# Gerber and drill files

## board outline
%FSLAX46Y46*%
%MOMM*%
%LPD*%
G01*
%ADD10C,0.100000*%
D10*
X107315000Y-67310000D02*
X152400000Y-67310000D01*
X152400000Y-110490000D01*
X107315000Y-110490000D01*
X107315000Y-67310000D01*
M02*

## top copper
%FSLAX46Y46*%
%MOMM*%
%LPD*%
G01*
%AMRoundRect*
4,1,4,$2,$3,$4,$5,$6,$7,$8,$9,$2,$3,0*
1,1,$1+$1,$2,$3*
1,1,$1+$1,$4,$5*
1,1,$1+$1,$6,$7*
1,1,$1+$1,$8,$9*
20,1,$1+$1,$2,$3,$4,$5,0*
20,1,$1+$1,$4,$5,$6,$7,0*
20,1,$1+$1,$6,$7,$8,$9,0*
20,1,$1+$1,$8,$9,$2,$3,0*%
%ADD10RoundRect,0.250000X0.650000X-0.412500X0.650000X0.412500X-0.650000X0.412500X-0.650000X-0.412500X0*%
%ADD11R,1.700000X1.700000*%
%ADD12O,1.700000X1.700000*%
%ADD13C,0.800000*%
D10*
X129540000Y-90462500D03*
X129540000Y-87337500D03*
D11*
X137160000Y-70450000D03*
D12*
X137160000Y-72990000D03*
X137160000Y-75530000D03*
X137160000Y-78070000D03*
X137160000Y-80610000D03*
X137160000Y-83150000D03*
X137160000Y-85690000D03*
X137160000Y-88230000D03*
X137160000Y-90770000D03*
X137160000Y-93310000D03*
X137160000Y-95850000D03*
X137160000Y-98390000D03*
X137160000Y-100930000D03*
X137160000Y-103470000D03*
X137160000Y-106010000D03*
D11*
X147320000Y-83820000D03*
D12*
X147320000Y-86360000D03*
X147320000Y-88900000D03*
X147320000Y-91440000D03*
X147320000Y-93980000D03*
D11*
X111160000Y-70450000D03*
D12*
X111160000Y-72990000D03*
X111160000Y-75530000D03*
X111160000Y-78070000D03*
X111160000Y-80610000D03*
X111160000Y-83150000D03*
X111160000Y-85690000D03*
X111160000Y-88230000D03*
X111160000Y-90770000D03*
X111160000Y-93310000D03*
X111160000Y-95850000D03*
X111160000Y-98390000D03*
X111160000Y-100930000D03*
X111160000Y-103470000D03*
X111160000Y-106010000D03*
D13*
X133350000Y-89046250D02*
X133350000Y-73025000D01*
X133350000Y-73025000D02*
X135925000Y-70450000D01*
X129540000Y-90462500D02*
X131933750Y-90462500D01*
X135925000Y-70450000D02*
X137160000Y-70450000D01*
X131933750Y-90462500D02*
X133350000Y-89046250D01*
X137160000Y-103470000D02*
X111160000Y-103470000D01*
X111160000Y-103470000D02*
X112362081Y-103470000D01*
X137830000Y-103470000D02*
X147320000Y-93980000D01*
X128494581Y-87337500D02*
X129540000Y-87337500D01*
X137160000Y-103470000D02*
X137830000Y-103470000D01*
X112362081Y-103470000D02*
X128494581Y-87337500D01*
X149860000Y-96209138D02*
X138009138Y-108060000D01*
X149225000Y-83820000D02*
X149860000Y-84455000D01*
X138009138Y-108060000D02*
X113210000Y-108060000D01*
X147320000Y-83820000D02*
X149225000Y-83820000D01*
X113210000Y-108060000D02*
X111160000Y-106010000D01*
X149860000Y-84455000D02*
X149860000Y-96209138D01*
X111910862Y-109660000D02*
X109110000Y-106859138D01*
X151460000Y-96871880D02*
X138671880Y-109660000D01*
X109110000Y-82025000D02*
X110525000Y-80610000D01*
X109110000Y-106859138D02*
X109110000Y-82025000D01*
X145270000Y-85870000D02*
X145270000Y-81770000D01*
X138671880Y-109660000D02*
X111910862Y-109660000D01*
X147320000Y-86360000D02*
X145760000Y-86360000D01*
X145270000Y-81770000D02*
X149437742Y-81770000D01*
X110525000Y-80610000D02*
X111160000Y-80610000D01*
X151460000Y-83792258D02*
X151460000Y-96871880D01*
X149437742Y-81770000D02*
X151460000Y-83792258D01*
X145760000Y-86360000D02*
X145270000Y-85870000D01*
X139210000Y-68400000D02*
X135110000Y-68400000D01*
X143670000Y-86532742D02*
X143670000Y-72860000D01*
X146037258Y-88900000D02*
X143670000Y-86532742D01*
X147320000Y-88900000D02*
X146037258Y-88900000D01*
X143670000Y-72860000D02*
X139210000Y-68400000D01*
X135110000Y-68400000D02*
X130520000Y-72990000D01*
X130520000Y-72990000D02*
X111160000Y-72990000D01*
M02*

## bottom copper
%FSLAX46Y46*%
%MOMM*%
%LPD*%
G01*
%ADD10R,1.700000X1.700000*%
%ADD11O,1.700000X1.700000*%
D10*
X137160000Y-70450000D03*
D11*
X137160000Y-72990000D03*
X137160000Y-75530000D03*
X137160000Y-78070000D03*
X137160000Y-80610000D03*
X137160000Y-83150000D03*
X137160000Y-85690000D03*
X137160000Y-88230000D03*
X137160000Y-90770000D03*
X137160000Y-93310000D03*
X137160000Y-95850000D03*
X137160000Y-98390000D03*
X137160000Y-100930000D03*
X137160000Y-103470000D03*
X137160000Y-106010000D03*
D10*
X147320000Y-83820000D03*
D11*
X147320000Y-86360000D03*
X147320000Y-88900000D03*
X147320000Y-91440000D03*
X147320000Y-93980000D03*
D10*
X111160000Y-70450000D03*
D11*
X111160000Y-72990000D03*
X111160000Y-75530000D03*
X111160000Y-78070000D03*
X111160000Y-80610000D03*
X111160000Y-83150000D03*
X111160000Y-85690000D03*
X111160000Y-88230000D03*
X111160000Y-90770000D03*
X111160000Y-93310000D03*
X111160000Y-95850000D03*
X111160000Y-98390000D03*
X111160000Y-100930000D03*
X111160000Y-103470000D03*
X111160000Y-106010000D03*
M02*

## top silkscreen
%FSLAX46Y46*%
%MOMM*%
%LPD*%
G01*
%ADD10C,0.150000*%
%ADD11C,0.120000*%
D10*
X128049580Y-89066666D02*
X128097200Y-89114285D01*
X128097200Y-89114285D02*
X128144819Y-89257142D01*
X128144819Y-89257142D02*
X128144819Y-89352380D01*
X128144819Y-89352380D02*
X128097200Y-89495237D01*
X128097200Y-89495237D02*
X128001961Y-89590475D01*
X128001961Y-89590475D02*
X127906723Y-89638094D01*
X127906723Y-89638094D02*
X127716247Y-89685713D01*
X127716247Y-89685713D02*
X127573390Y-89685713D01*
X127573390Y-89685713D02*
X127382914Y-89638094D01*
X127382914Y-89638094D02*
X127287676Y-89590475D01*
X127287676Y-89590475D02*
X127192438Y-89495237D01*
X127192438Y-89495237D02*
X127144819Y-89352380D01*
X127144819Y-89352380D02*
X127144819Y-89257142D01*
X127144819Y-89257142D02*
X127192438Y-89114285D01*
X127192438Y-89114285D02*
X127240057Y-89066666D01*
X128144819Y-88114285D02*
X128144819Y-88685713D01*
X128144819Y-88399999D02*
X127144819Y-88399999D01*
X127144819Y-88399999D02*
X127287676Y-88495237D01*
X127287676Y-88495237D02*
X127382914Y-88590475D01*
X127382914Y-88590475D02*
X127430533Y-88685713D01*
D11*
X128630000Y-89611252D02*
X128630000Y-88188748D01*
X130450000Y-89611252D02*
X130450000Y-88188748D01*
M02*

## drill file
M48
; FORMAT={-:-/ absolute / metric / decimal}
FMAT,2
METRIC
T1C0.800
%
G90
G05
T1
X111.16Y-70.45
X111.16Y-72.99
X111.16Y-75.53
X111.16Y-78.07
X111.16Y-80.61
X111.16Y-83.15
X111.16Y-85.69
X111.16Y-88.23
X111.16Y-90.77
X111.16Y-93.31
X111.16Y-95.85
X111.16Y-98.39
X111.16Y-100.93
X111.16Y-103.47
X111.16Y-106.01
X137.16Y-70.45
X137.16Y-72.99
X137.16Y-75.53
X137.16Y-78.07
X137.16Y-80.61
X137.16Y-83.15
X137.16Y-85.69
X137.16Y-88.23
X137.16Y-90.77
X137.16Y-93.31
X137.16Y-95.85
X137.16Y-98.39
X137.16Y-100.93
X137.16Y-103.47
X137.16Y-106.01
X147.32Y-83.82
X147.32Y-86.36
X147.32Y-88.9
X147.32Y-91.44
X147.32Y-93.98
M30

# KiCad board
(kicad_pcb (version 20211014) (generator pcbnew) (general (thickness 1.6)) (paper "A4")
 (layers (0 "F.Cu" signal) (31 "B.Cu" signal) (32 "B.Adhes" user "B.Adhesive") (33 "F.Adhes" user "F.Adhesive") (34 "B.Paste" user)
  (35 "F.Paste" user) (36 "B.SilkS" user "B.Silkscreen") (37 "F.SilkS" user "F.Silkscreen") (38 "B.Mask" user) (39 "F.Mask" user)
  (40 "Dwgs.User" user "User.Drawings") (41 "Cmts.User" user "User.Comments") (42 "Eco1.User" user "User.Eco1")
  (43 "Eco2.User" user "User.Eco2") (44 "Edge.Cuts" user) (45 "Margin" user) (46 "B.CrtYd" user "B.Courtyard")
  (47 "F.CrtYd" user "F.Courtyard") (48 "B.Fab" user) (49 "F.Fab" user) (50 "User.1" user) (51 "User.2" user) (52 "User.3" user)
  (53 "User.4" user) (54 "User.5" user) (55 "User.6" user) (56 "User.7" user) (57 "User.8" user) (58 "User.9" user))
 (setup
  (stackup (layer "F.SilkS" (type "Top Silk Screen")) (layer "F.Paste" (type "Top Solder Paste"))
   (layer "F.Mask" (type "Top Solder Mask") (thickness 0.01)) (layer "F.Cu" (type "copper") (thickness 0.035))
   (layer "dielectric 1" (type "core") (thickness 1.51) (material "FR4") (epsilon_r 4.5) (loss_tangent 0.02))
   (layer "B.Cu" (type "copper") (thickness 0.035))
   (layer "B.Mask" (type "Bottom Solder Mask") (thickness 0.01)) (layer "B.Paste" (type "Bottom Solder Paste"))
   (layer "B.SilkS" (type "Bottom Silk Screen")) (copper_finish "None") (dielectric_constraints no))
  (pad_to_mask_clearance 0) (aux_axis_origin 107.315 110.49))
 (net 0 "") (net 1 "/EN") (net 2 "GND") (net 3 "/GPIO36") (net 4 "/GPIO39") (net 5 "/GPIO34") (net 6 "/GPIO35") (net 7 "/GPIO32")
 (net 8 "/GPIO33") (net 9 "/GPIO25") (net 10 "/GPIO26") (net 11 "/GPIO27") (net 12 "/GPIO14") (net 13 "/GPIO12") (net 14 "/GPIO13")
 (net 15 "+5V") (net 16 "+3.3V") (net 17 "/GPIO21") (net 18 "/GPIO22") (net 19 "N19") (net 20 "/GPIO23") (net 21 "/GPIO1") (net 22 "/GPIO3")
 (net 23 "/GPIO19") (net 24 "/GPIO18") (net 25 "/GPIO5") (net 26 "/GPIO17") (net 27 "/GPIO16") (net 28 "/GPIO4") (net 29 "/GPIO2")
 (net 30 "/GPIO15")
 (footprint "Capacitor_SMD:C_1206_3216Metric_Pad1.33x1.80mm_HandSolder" (layer "F.Cu") (at 129.54 88.9 90)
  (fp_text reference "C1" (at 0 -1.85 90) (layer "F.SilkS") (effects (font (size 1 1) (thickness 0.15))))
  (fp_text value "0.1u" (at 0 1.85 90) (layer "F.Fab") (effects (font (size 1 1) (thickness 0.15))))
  (fp_line (start -0.711252 -0.91) (end 0.711252 -0.91) (layer "F.SilkS") (width 0.12))
  (fp_line (start -0.711252 0.91) (end 0.711252 0.91) (layer "F.SilkS") (width 0.12))
  (pad "1" smd roundrect (at -1.5625 0 90) (size 1.325 1.8) (layers "F.Cu" "F.Paste" "F.Mask") (roundrect_rratio 0.1886792453) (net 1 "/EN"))
  (pad "2" smd roundrect (at 1.5625 0 90) (size 1.325 1.8) (layers "F.Cu" "F.Paste" "F.Mask") (roundrect_rratio 0.1886792453) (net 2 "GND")))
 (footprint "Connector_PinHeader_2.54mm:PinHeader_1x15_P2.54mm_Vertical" (layer "B.Cu") (at 137.16 70.45 180)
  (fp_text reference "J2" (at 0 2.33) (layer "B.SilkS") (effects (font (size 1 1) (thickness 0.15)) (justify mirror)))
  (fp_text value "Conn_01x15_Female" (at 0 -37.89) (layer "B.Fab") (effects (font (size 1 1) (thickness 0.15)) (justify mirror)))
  (pad "1" thru_hole rect (at 0 0 180) (size 1.7 1.7) (drill 0.8) (layers *.Cu *.Mask) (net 1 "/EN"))
  (pad "2" thru_hole oval (at 0 -2.54 180) (size 1.7 1.7) (drill 0.8) (layers *.Cu *.Mask) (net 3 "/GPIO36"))
  (pad "3" thru_hole oval (at 0 -5.08 180) (size 1.7 1.7) (drill 0.8) (layers *.Cu *.Mask) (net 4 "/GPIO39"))
  (pad "4" thru_hole oval (at 0 -7.62 180) (size 1.7 1.7) (drill 0.8) (layers *.Cu *.Mask) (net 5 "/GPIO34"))
  (pad "5" thru_hole oval (at 0 -10.16 180) (size 1.7 1.7) (drill 0.8) (layers *.Cu *.Mask) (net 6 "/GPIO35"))
  (pad "6" thru_hole oval (at 0 -12.7 180) (size 1.7 1.7) (drill 0.8) (layers *.Cu *.Mask) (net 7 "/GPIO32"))
  (pad "7" thru_hole oval (at 0 -15.24 180) (size 1.7 1.7) (drill 0.8) (layers *.Cu *.Mask) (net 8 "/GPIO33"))
  (pad "8" thru_hole oval (at 0 -17.78 180) (size 1.7 1.7) (drill 0.8) (layers *.Cu *.Mask) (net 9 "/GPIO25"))
  (pad "9" thru_hole oval (at 0 -20.32 180) (size 1.7 1.7) (drill 0.8) (layers *.Cu *.Mask) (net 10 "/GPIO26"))
  (pad "10" thru_hole oval (at 0 -22.86 180) (size 1.7 1.7) (drill 0.8) (layers *.Cu *.Mask) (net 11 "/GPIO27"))
  (pad "11" thru_hole oval (at 0 -25.4 180) (size 1.7 1.7) (drill 0.8) (layers *.Cu *.Mask) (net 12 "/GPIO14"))
  (pad "12" thru_hole oval (at 0 -27.94 180) (size 1.7 1.7) (drill 0.8) (layers *.Cu *.Mask) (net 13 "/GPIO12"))
  (pad "13" thru_hole oval (at 0 -30.48 180) (size 1.7 1.7) (drill 0.8) (layers *.Cu *.Mask) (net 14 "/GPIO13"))
  (pad "14" thru_hole oval (at 0 -33.02 180) (size 1.7 1.7) (drill 0.8) (layers *.Cu *.Mask) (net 2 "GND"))
  (pad "15" thru_hole oval (at 0 -35.56 180) (size 1.7 1.7) (drill 0.8) (layers *.Cu *.Mask) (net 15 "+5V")))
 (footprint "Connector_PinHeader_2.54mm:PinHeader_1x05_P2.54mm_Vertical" (layer "B.Cu") (at 147.32 83.82 180)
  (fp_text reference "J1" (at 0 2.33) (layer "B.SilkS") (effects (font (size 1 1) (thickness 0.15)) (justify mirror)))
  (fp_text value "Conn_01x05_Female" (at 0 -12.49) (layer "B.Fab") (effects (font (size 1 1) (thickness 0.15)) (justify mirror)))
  (pad "1" thru_hole rect (at 0 0 180) (size 1.7 1.7) (drill 0.8) (layers *.Cu *.Mask) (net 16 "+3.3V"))
  (pad "2" thru_hole oval (at 0 -2.54 180) (size 1.7 1.7) (drill 0.8) (layers *.Cu *.Mask) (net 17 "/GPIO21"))
  (pad "3" thru_hole oval (at 0 -5.08 180) (size 1.7 1.7) (drill 0.8) (layers *.Cu *.Mask) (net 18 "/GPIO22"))
  (pad "4" thru_hole oval (at 0 -7.62 180) (size 1.7 1.7) (drill 0.8) (layers *.Cu *.Mask) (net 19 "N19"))
  (pad "5" thru_hole oval (at 0 -10.16 180) (size 1.7 1.7) (drill 0.8) (layers *.Cu *.Mask) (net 2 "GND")))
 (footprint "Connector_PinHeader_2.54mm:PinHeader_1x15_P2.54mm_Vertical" (layer "B.Cu") (at 111.16 70.45 180)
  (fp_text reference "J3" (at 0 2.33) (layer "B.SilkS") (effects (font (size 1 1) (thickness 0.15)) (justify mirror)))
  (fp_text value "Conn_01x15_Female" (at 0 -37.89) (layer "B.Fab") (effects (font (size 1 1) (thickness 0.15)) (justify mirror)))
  (pad "1" thru_hole rect (at 0 0 180) (size 1.7 1.7) (drill 0.8) (layers *.Cu *.Mask) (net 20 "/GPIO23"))
  (pad "2" thru_hole oval (at 0 -2.54 180) (size 1.7 1.7) (drill 0.8) (layers *.Cu *.Mask) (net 18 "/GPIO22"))
  (pad "3" thru_hole oval (at 0 -5.08 180) (size 1.7 1.7) (drill 0.8) (layers *.Cu *.Mask) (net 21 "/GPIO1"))
  (pad "4" thru_hole oval (at 0 -7.62 180) (size 1.7 1.7) (drill 0.8) (layers *.Cu *.Mask) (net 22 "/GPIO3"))
  (pad "5" thru_hole oval (at 0 -10.16 180) (size 1.7 1.7) (drill 0.8) (layers *.Cu *.Mask) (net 17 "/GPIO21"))
  (pad "6" thru_hole oval (at 0 -12.7 180) (size 1.7 1.7) (drill 0.8) (layers *.Cu *.Mask) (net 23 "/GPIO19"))
  (pad "7" thru_hole oval (at 0 -15.24 180) (size 1.7 1.7) (drill 0.8) (layers *.Cu *.Mask) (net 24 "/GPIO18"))
  (pad "8" thru_hole oval (at 0 -17.78 180) (size 1.7 1.7) (drill 0.8) (layers *.Cu *.Mask) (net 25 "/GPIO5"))
  (pad "9" thru_hole oval (at 0 -20.32 180) (size 1.7 1.7) (drill 0.8) (layers *.Cu *.Mask) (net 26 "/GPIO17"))
  (pad "10" thru_hole oval (at 0 -22.86 180) (size 1.7 1.7) (drill 0.8) (layers *.Cu *.Mask) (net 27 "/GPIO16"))
  (pad "11" thru_hole oval (at 0 -25.4 180) (size 1.7 1.7) (drill 0.8) (layers *.Cu *.Mask) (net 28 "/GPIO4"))
  (pad "12" thru_hole oval (at 0 -27.94 180) (size 1.7 1.7) (drill 0.8) (layers *.Cu *.Mask) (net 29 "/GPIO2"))
  (pad "13" thru_hole oval (at 0 -30.48 180) (size 1.7 1.7) (drill 0.8) (layers *.Cu *.Mask) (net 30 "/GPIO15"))
  (pad "14" thru_hole oval (at 0 -33.02 180) (size 1.7 1.7) (drill 0.8) (layers *.Cu *.Mask) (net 2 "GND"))
  (pad "15" thru_hole oval (at 0 -35.56 180) (size 1.7 1.7) (drill 0.8) (layers *.Cu *.Mask) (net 16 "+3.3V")))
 (gr_rect (start 107.315 67.31) (end 152.4 110.49) (layer "Edge.Cuts") (width 0.1) (fill none))
 (segment (start 133.35 89.04625) (end 133.35 73.025) (width 0.8) (layer "F.Cu") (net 1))
 (segment (start 133.35 73.025) (end 135.925 70.45) (width 0.8) (layer "F.Cu") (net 1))
 (segment (start 129.54 90.4625) (end 131.93375 90.4625) (width 0.8) (layer "F.Cu") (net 1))
 (segment (start 135.925 70.45) (end 137.16 70.45) (width 0.8) (layer "F.Cu") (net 1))
 (segment (start 131.93375 90.4625) (end 133.35 89.04625) (width 0.8) (layer "F.Cu") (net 1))
 (segment (start 137.16 103.47) (end 111.16 103.47) (width 0.8) (layer "F.Cu") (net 2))
 (segment (start 111.16 103.47) (end 112.362081 103.47) (width 0.8) (layer "F.Cu") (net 2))
 (segment (start 137.83 103.47) (end 147.32 93.98) (width 0.8) (layer "F.Cu") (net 2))
 (segment (start 128.494581 87.3375) (end 129.54 87.3375) (width 0.8) (layer "F.Cu") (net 2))
 (segment (start 137.16 103.47) (end 137.83 103.47) (width 0.8) (layer "F.Cu") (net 2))
 (segment (start 112.362081 103.47) (end 128.494581 87.3375) (width 0.8) (layer "F.Cu") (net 2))
 (segment (start 149.86 96.209138) (end 138.009138 108.06) (width 0.8) (layer "F.Cu") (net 16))
 (segment (start 149.225 83.82) (end 149.86 84.455) (width 0.8) (layer "F.Cu") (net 16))
 (segment (start 138.009138 108.06) (end 113.21 108.06) (width 0.8) (layer "F.Cu") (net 16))
 (segment (start 147.32 83.82) (end 149.225 83.82) (width 0.8) (layer "F.Cu") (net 16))
 (segment (start 113.21 108.06) (end 111.16 106.01) (width 0.8) (layer "F.Cu") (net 16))
 (segment (start 149.86 84.455) (end 149.86 96.209138) (width 0.8) (layer "F.Cu") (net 16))
 (segment (start 111.910862 109.66) (end 109.11 106.859138) (width 0.8) (layer "F.Cu") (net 17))
 (segment (start 151.46 96.87188) (end 138.67188 109.66) (width 0.8) (layer "F.Cu") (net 17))
 (segment (start 109.11 82.025) (end 110.525 80.61) (width 0.8) (layer "F.Cu") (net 17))
 (segment (start 109.11 106.859138) (end 109.11 82.025) (width 0.8) (layer "F.Cu") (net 17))
 (segment (start 145.27 85.87) (end 145.27 81.77) (width 0.8) (layer "F.Cu") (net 17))
 (segment (start 138.67188 109.66) (end 111.910862 109.66) (width 0.8) (layer "F.Cu") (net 17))
 (segment (start 147.32 86.36) (end 145.76 86.36) (width 0.8) (layer "F.Cu") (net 17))
 (segment (start 145.27 81.77) (end 149.437742 81.77) (width 0.8) (layer "F.Cu") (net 17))
 (segment (start 110.525 80.61) (end 111.16 80.61) (width 0.8) (layer "F.Cu") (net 17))
 (segment (start 151.46 83.792258) (end 151.46 96.87188) (width 0.8) (layer "F.Cu") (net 17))
 (segment (start 149.437742 81.77) (end 151.46 83.792258) (width 0.8) (layer "F.Cu") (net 17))
 (segment (start 145.76 86.36) (end 145.27 85.87) (width 0.8) (layer "F.Cu") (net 17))
 (segment (start 139.21 68.4) (end 135.11 68.4) (width 0.8) (layer "F.Cu") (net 18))
 (segment (start 143.67 86.532742) (end 143.67 72.86) (width 0.8) (layer "F.Cu") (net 18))
 (segment (start 146.037258 88.9) (end 143.67 86.532742) (width 0.8) (layer "F.Cu") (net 18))
 (segment (start 147.32 88.9) (end 146.037258 88.9) (width 0.8) (layer "F.Cu") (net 18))
 (segment (start 143.67 72.86) (end 139.21 68.4) (width 0.8) (layer "F.Cu") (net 18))
 (segment (start 135.11 68.4) (end 130.52 72.99) (width 0.8) (layer "F.Cu") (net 18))
 (segment (start 130.52 72.99) (end 111.16 72.99) (width 0.8) (layer "F.Cu") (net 18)))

